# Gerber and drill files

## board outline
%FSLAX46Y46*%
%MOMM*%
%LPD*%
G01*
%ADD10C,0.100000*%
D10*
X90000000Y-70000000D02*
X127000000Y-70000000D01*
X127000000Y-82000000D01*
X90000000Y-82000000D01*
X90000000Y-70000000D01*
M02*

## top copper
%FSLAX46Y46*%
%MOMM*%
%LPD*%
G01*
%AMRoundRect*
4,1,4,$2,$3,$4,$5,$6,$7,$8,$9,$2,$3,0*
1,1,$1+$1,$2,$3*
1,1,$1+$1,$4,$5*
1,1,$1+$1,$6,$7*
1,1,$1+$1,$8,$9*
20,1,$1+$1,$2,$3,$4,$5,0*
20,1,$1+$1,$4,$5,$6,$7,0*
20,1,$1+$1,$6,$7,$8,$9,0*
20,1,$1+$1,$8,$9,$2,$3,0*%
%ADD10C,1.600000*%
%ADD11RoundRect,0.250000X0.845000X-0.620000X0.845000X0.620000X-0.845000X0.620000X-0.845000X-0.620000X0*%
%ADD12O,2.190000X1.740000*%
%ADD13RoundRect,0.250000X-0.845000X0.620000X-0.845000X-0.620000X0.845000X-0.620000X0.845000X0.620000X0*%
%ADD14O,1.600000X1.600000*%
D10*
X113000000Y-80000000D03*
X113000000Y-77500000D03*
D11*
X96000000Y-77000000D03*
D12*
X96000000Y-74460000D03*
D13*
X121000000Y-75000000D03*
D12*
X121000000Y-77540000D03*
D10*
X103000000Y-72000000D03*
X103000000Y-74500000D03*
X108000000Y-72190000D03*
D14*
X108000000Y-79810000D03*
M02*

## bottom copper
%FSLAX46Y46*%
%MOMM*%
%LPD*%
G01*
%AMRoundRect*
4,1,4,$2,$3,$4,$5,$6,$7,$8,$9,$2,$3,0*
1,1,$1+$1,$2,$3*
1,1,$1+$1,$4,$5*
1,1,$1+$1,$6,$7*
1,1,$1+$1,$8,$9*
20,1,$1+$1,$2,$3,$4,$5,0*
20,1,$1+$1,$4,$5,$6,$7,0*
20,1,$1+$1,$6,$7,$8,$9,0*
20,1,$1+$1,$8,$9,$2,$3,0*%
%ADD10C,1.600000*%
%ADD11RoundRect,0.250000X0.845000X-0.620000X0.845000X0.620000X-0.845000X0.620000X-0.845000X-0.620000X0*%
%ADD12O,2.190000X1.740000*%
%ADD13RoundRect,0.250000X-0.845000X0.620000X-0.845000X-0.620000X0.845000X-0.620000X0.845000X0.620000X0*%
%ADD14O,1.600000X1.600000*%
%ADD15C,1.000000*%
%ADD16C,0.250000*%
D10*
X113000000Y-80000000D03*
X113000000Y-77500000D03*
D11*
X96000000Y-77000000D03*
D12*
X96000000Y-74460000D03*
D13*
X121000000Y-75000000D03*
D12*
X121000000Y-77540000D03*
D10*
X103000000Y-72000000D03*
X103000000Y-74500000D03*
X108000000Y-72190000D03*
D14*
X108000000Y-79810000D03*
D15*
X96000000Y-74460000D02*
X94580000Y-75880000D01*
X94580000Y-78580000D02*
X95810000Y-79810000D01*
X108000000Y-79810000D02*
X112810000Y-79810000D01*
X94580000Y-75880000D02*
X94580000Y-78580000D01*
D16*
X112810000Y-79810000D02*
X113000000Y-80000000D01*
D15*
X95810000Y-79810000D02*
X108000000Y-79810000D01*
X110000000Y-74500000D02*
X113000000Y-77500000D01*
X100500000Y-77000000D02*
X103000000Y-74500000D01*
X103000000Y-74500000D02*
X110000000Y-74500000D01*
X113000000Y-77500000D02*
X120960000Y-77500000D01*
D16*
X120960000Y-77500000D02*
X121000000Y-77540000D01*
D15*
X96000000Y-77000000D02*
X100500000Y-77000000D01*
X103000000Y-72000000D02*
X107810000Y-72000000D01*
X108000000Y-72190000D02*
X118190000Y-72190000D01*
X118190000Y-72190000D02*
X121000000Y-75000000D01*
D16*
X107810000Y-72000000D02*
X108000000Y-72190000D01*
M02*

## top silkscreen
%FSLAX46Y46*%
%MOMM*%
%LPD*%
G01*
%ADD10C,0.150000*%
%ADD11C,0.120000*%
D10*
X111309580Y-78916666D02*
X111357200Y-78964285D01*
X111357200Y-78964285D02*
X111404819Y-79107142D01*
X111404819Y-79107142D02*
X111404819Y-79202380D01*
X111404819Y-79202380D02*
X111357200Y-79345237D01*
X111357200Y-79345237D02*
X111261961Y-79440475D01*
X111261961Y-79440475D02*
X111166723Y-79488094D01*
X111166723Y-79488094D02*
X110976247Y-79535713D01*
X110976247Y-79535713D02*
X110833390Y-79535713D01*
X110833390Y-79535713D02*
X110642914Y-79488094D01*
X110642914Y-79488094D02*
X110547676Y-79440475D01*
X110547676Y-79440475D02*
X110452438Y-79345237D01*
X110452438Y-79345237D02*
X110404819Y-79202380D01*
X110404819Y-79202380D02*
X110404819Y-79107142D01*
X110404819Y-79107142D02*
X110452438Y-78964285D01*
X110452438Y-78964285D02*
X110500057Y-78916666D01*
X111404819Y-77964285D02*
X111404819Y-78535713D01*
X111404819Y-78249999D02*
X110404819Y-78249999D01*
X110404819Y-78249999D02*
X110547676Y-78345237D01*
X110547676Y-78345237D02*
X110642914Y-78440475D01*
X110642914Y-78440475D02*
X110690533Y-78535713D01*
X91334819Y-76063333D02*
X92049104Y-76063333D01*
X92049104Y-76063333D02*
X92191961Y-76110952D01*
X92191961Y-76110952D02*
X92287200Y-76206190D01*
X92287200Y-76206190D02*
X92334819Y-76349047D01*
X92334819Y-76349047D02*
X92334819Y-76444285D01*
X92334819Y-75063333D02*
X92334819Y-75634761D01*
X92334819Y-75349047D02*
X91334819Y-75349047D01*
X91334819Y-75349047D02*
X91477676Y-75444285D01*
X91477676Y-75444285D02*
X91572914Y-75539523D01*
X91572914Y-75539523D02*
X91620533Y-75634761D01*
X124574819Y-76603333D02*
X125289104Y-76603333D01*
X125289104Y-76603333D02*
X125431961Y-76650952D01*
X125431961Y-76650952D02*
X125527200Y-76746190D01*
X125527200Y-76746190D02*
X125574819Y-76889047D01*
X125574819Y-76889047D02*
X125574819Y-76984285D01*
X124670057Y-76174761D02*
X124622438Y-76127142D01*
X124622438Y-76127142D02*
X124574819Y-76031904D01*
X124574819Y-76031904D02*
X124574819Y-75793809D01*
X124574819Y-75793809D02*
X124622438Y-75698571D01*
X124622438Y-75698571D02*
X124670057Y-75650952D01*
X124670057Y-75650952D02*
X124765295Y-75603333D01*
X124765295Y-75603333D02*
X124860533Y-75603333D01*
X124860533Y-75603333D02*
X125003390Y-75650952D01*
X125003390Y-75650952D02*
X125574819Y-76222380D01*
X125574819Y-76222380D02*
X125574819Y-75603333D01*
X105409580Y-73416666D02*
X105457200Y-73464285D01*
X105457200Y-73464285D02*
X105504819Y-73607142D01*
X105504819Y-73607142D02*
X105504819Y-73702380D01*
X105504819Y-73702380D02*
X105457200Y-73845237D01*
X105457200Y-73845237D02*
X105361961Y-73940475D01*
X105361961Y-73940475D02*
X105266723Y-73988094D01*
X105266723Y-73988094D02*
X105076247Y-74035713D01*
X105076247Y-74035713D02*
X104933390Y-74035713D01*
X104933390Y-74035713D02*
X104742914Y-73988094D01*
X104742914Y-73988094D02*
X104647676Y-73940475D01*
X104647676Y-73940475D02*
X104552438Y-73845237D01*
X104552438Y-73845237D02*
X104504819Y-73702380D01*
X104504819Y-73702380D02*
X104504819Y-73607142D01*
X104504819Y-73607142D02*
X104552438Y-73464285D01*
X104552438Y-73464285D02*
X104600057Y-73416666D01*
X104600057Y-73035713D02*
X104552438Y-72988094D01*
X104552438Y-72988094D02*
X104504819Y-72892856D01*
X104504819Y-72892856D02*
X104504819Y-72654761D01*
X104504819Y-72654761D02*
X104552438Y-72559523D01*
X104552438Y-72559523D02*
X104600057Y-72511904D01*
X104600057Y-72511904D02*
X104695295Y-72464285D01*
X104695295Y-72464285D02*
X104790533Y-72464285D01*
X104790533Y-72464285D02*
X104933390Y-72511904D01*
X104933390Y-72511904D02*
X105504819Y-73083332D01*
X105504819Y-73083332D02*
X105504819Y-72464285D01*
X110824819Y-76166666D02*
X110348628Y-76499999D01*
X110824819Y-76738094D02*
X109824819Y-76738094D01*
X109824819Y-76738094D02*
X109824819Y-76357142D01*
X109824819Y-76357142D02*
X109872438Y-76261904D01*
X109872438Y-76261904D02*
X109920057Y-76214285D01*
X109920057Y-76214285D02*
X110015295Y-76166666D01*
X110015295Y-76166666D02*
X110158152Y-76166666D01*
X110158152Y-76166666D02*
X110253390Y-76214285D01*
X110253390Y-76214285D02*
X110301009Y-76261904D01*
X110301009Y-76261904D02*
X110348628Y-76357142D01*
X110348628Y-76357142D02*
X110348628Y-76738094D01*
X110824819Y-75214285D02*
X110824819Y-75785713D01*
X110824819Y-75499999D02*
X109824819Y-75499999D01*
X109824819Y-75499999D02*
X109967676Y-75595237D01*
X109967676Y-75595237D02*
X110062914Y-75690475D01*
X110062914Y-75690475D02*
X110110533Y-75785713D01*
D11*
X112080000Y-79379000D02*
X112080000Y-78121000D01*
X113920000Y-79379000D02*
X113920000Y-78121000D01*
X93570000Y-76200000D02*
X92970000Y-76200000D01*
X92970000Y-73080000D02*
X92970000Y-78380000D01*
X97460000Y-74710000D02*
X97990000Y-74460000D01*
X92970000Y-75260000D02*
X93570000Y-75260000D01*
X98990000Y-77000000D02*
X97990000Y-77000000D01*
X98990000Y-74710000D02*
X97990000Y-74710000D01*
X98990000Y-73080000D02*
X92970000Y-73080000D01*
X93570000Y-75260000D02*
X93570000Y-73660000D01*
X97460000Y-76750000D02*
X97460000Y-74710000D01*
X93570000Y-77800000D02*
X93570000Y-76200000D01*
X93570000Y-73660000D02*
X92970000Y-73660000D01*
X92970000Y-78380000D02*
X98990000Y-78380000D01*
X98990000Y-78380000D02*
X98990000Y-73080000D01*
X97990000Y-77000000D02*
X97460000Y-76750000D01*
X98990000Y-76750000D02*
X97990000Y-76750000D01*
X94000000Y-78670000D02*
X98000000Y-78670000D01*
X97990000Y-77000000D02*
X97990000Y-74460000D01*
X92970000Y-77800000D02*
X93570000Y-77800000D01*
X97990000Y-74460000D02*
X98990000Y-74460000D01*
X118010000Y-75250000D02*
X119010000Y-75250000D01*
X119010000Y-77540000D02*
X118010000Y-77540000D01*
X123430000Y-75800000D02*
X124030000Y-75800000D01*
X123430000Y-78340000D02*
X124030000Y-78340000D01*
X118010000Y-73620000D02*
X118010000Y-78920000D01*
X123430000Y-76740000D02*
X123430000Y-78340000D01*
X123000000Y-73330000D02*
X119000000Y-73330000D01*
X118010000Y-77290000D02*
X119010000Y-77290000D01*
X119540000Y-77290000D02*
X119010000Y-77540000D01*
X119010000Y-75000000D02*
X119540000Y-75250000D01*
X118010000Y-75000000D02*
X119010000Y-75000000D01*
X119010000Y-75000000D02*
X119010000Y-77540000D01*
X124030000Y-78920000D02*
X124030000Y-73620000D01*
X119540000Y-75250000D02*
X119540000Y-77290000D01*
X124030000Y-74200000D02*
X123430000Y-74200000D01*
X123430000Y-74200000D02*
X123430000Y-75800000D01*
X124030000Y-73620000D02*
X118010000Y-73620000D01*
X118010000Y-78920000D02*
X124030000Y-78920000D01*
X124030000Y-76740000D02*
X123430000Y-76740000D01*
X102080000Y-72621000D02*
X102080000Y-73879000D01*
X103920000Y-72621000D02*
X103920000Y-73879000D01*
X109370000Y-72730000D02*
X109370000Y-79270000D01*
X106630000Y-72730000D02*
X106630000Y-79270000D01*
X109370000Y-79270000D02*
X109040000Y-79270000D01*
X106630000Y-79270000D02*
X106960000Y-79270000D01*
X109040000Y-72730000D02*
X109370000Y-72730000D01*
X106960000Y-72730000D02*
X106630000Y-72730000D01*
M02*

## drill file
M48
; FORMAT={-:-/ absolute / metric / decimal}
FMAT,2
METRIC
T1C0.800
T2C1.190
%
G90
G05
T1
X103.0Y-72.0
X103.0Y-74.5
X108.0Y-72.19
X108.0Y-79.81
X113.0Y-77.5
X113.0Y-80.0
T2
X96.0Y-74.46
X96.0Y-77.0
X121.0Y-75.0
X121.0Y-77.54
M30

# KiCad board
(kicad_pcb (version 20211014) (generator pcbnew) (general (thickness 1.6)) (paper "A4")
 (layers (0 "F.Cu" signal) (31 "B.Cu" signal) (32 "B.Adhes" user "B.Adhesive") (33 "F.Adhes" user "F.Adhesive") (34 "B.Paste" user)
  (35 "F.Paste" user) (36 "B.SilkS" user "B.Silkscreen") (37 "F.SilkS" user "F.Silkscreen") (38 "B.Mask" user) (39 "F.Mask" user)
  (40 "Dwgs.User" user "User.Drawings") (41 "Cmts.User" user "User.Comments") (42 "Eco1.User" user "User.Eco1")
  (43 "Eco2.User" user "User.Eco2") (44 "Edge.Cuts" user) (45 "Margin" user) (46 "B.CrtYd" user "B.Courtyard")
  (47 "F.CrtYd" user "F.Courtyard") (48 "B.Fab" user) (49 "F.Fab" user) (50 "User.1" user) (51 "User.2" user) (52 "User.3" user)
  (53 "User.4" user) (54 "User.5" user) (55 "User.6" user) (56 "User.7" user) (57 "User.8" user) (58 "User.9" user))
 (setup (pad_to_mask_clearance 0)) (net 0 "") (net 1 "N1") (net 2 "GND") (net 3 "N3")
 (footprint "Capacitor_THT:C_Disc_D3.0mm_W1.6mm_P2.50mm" (layer "F.Cu") (at 113 80 90)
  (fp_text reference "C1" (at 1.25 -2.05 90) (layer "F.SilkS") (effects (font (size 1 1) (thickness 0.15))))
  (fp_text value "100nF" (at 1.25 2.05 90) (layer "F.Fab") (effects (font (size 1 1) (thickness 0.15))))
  (fp_line (start 0.621 -0.92) (end 1.879 -0.92) (layer "F.SilkS") (width 0.12))
  (fp_line (start 0.621 0.92) (end 1.879 0.92) (layer "F.SilkS") (width 0.12))
  (pad "1" thru_hole circle (at 0 0 90) (size 1.6 1.6) (drill 0.8) (layers *.Cu *.Mask) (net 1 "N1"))
  (pad "2" thru_hole circle (at 2.5 0 90) (size 1.6 1.6) (drill 0.8) (layers *.Cu *.Mask) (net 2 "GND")))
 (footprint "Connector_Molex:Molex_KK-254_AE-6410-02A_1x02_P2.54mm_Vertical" (layer "F.Cu") (at 96 77 90)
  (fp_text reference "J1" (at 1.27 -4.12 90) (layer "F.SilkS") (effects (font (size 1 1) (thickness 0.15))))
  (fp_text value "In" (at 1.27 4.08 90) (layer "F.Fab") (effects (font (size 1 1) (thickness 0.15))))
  (fp_line (start 0.8 -2.43) (end 0.8 -3.03) (layer "F.SilkS") (width 0.12))
  (fp_line (start 3.92 -3.03) (end -1.38 -3.03) (layer "F.SilkS") (width 0.12))
  (fp_line (start 2.29 1.46) (end 2.54 1.99) (layer "F.SilkS") (width 0.12))
  (fp_line (start 1.74 -3.03) (end 1.74 -2.43) (layer "F.SilkS") (width 0.12))
  (fp_line (start 0 2.99) (end 0 1.99) (layer "F.SilkS") (width 0.12))
  (fp_line (start 2.29 2.99) (end 2.29 1.99) (layer "F.SilkS") (width 0.12))
  (fp_line (start 3.92 2.99) (end 3.92 -3.03) (layer "F.SilkS") (width 0.12))
  (fp_line (start 1.74 -2.43) (end 3.34 -2.43) (layer "F.SilkS") (width 0.12))
  (fp_line (start 0.25 1.46) (end 2.29 1.46) (layer "F.SilkS") (width 0.12))
  (fp_line (start -0.8 -2.43) (end 0.8 -2.43) (layer "F.SilkS") (width 0.12))
  (fp_line (start 3.34 -2.43) (end 3.34 -3.03) (layer "F.SilkS") (width 0.12))
  (fp_line (start -1.38 -3.03) (end -1.38 2.99) (layer "F.SilkS") (width 0.12))
  (fp_line (start -1.38 2.99) (end 3.92 2.99) (layer "F.SilkS") (width 0.12))
  (fp_line (start 0 1.99) (end 0.25 1.46) (layer "F.SilkS") (width 0.12))
  (fp_line (start 0.25 2.99) (end 0.25 1.99) (layer "F.SilkS") (width 0.12))
  (fp_line (start -1.67 -2) (end -1.67 2) (layer "F.SilkS") (width 0.12))
  (fp_line (start 0 1.99) (end 2.54 1.99) (layer "F.SilkS") (width 0.12))
  (fp_line (start -0.8 -3.03) (end -0.8 -2.43) (layer "F.SilkS") (width 0.12))
  (fp_line (start 2.54 1.99) (end 2.54 2.99) (layer "F.SilkS") (width 0.12))
  (pad "1" thru_hole roundrect (at 0 0 90) (size 1.74 2.19) (drill 1.19) (layers *.Cu *.Mask) (roundrect_rratio 0.143678) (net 2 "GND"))
  (pad "2" thru_hole oval (at 2.54 0 90) (size 1.74 2.19) (drill 1.19) (layers *.Cu *.Mask) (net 1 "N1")))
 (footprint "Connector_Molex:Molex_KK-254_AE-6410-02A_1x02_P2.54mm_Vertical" (layer "F.Cu") (at 121 75 -90)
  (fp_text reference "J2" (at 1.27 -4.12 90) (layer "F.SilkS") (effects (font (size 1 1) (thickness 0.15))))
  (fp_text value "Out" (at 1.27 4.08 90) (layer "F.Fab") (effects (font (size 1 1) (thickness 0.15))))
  (fp_line (start 0.25 2.99) (end 0.25 1.99) (layer "F.SilkS") (width 0.12))
  (fp_line (start 2.54 1.99) (end 2.54 2.99) (layer "F.SilkS") (width 0.12))
  (fp_line (start 0.8 -2.43) (end 0.8 -3.03) (layer "F.SilkS") (width 0.12))
  (fp_line (start 3.34 -2.43) (end 3.34 -3.03) (layer "F.SilkS") (width 0.12))
  (fp_line (start -1.38 2.99) (end 3.92 2.99) (layer "F.SilkS") (width 0.12))
  (fp_line (start 1.74 -2.43) (end 3.34 -2.43) (layer "F.SilkS") (width 0.12))
  (fp_line (start -1.67 -2) (end -1.67 2) (layer "F.SilkS") (width 0.12))
  (fp_line (start 2.29 2.99) (end 2.29 1.99) (layer "F.SilkS") (width 0.12))
  (fp_line (start 2.29 1.46) (end 2.54 1.99) (layer "F.SilkS") (width 0.12))
  (fp_line (start 0 1.99) (end 0.25 1.46) (layer "F.SilkS") (width 0.12))
  (fp_line (start 0 2.99) (end 0 1.99) (layer "F.SilkS") (width 0.12))
  (fp_line (start 0 1.99) (end 2.54 1.99) (layer "F.SilkS") (width 0.12))
  (fp_line (start 3.92 -3.03) (end -1.38 -3.03) (layer "F.SilkS") (width 0.12))
  (fp_line (start 0.25 1.46) (end 2.29 1.46) (layer "F.SilkS") (width 0.12))
  (fp_line (start -0.8 -3.03) (end -0.8 -2.43) (layer "F.SilkS") (width 0.12))
  (fp_line (start -0.8 -2.43) (end 0.8 -2.43) (layer "F.SilkS") (width 0.12))
  (fp_line (start -1.38 -3.03) (end -1.38 2.99) (layer "F.SilkS") (width 0.12))
  (fp_line (start 3.92 2.99) (end 3.92 -3.03) (layer "F.SilkS") (width 0.12))
  (fp_line (start 1.74 -3.03) (end 1.74 -2.43) (layer "F.SilkS") (width 0.12))
  (pad "1" thru_hole roundrect (at 0 0 270) (size 1.74 2.19) (drill 1.19) (layers *.Cu *.Mask) (roundrect_rratio 0.143678) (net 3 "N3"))
  (pad "2" thru_hole oval (at 2.54 0 270) (size 1.74 2.19) (drill 1.19) (layers *.Cu *.Mask) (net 2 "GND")))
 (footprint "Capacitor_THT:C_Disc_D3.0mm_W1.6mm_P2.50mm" (layer "F.Cu") (at 103 72 -90)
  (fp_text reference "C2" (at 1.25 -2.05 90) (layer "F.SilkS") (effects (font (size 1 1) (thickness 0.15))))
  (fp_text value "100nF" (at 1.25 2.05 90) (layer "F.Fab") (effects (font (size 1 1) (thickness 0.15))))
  (fp_line (start 0.621 0.92) (end 1.879 0.92) (layer "F.SilkS") (width 0.12))
  (fp_line (start 0.621 -0.92) (end 1.879 -0.92) (layer "F.SilkS") (width 0.12))
  (pad "1" thru_hole circle (at 0 0 270) (size 1.6 1.6) (drill 0.8) (layers *.Cu *.Mask) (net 3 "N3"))
  (pad "2" thru_hole circle (at 2.5 0 270) (size 1.6 1.6) (drill 0.8) (layers *.Cu *.Mask) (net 2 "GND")))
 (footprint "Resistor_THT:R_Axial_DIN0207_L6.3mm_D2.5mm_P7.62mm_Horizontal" (layer "F.Cu") (at 108 72.19 -90)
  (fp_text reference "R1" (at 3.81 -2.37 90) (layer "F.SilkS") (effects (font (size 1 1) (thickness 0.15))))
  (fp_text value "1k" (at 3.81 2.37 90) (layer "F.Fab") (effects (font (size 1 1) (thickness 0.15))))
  (fp_line (start 0.54 -1.37) (end 7.08 -1.37) (layer "F.SilkS") (width 0.12))
  (fp_line (start 0.54 1.37) (end 7.08 1.37) (layer "F.SilkS") (width 0.12))
  (fp_line (start 7.08 -1.37) (end 7.08 -1.04) (layer "F.SilkS") (width 0.12))
  (fp_line (start 7.08 1.37) (end 7.08 1.04) (layer "F.SilkS") (width 0.12))
  (fp_line (start 0.54 -1.04) (end 0.54 -1.37) (layer "F.SilkS") (width 0.12))
  (fp_line (start 0.54 1.04) (end 0.54 1.37) (layer "F.SilkS") (width 0.12))
  (pad "1" thru_hole circle (at 0 0 270) (size 1.6 1.6) (drill 0.8) (layers *.Cu *.Mask) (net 3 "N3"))
  (pad "2" thru_hole oval (at 7.62 0 270) (size 1.6 1.6) (drill 0.8) (layers *.Cu *.Mask) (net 1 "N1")))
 (gr_rect (start 90 70) (end 127 82) (layer "Edge.Cuts") (width 0.1) (fill none))
 (segment (start 96 74.46) (end 94.58 75.88) (width 1) (layer "B.Cu") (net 1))
 (segment (start 94.58 78.58) (end 95.81 79.81) (width 1) (layer "B.Cu") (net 1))
 (segment (start 108 79.81) (end 112.81 79.81) (width 1) (layer "B.Cu") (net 1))
 (segment (start 94.58 75.88) (end 94.58 78.58) (width 1) (layer "B.Cu") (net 1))
 (segment (start 112.81 79.81) (end 113 80) (width 0.25) (layer "B.Cu") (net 1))
 (segment (start 95.81 79.81) (end 108 79.81) (width 1) (layer "B.Cu") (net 1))
 (segment (start 110 74.5) (end 113 77.5) (width 1) (layer "B.Cu") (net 2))
 (segment (start 100.5 77) (end 103 74.5) (width 1) (layer "B.Cu") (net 2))
 (segment (start 103 74.5) (end 110 74.5) (width 1) (layer "B.Cu") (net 2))
 (segment (start 113 77.5) (end 120.96 77.5) (width 1) (layer "B.Cu") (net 2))
 (segment (start 120.96 77.5) (end 121 77.54) (width 0.25) (layer "B.Cu") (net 2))
 (segment (start 96 77) (end 100.5 77) (width 1) (layer "B.Cu") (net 2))
 (segment (start 103 72) (end 107.81 72) (width 1) (layer "B.Cu") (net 3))
 (segment (start 108 72.19) (end 118.19 72.19) (width 1) (layer "B.Cu") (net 3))
 (segment (start 118.19 72.19) (end 121 75) (width 1) (layer "B.Cu") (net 3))
 (segment (start 107.81 72) (end 108 72.19) (width 0.25) (layer "B.Cu") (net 3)))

